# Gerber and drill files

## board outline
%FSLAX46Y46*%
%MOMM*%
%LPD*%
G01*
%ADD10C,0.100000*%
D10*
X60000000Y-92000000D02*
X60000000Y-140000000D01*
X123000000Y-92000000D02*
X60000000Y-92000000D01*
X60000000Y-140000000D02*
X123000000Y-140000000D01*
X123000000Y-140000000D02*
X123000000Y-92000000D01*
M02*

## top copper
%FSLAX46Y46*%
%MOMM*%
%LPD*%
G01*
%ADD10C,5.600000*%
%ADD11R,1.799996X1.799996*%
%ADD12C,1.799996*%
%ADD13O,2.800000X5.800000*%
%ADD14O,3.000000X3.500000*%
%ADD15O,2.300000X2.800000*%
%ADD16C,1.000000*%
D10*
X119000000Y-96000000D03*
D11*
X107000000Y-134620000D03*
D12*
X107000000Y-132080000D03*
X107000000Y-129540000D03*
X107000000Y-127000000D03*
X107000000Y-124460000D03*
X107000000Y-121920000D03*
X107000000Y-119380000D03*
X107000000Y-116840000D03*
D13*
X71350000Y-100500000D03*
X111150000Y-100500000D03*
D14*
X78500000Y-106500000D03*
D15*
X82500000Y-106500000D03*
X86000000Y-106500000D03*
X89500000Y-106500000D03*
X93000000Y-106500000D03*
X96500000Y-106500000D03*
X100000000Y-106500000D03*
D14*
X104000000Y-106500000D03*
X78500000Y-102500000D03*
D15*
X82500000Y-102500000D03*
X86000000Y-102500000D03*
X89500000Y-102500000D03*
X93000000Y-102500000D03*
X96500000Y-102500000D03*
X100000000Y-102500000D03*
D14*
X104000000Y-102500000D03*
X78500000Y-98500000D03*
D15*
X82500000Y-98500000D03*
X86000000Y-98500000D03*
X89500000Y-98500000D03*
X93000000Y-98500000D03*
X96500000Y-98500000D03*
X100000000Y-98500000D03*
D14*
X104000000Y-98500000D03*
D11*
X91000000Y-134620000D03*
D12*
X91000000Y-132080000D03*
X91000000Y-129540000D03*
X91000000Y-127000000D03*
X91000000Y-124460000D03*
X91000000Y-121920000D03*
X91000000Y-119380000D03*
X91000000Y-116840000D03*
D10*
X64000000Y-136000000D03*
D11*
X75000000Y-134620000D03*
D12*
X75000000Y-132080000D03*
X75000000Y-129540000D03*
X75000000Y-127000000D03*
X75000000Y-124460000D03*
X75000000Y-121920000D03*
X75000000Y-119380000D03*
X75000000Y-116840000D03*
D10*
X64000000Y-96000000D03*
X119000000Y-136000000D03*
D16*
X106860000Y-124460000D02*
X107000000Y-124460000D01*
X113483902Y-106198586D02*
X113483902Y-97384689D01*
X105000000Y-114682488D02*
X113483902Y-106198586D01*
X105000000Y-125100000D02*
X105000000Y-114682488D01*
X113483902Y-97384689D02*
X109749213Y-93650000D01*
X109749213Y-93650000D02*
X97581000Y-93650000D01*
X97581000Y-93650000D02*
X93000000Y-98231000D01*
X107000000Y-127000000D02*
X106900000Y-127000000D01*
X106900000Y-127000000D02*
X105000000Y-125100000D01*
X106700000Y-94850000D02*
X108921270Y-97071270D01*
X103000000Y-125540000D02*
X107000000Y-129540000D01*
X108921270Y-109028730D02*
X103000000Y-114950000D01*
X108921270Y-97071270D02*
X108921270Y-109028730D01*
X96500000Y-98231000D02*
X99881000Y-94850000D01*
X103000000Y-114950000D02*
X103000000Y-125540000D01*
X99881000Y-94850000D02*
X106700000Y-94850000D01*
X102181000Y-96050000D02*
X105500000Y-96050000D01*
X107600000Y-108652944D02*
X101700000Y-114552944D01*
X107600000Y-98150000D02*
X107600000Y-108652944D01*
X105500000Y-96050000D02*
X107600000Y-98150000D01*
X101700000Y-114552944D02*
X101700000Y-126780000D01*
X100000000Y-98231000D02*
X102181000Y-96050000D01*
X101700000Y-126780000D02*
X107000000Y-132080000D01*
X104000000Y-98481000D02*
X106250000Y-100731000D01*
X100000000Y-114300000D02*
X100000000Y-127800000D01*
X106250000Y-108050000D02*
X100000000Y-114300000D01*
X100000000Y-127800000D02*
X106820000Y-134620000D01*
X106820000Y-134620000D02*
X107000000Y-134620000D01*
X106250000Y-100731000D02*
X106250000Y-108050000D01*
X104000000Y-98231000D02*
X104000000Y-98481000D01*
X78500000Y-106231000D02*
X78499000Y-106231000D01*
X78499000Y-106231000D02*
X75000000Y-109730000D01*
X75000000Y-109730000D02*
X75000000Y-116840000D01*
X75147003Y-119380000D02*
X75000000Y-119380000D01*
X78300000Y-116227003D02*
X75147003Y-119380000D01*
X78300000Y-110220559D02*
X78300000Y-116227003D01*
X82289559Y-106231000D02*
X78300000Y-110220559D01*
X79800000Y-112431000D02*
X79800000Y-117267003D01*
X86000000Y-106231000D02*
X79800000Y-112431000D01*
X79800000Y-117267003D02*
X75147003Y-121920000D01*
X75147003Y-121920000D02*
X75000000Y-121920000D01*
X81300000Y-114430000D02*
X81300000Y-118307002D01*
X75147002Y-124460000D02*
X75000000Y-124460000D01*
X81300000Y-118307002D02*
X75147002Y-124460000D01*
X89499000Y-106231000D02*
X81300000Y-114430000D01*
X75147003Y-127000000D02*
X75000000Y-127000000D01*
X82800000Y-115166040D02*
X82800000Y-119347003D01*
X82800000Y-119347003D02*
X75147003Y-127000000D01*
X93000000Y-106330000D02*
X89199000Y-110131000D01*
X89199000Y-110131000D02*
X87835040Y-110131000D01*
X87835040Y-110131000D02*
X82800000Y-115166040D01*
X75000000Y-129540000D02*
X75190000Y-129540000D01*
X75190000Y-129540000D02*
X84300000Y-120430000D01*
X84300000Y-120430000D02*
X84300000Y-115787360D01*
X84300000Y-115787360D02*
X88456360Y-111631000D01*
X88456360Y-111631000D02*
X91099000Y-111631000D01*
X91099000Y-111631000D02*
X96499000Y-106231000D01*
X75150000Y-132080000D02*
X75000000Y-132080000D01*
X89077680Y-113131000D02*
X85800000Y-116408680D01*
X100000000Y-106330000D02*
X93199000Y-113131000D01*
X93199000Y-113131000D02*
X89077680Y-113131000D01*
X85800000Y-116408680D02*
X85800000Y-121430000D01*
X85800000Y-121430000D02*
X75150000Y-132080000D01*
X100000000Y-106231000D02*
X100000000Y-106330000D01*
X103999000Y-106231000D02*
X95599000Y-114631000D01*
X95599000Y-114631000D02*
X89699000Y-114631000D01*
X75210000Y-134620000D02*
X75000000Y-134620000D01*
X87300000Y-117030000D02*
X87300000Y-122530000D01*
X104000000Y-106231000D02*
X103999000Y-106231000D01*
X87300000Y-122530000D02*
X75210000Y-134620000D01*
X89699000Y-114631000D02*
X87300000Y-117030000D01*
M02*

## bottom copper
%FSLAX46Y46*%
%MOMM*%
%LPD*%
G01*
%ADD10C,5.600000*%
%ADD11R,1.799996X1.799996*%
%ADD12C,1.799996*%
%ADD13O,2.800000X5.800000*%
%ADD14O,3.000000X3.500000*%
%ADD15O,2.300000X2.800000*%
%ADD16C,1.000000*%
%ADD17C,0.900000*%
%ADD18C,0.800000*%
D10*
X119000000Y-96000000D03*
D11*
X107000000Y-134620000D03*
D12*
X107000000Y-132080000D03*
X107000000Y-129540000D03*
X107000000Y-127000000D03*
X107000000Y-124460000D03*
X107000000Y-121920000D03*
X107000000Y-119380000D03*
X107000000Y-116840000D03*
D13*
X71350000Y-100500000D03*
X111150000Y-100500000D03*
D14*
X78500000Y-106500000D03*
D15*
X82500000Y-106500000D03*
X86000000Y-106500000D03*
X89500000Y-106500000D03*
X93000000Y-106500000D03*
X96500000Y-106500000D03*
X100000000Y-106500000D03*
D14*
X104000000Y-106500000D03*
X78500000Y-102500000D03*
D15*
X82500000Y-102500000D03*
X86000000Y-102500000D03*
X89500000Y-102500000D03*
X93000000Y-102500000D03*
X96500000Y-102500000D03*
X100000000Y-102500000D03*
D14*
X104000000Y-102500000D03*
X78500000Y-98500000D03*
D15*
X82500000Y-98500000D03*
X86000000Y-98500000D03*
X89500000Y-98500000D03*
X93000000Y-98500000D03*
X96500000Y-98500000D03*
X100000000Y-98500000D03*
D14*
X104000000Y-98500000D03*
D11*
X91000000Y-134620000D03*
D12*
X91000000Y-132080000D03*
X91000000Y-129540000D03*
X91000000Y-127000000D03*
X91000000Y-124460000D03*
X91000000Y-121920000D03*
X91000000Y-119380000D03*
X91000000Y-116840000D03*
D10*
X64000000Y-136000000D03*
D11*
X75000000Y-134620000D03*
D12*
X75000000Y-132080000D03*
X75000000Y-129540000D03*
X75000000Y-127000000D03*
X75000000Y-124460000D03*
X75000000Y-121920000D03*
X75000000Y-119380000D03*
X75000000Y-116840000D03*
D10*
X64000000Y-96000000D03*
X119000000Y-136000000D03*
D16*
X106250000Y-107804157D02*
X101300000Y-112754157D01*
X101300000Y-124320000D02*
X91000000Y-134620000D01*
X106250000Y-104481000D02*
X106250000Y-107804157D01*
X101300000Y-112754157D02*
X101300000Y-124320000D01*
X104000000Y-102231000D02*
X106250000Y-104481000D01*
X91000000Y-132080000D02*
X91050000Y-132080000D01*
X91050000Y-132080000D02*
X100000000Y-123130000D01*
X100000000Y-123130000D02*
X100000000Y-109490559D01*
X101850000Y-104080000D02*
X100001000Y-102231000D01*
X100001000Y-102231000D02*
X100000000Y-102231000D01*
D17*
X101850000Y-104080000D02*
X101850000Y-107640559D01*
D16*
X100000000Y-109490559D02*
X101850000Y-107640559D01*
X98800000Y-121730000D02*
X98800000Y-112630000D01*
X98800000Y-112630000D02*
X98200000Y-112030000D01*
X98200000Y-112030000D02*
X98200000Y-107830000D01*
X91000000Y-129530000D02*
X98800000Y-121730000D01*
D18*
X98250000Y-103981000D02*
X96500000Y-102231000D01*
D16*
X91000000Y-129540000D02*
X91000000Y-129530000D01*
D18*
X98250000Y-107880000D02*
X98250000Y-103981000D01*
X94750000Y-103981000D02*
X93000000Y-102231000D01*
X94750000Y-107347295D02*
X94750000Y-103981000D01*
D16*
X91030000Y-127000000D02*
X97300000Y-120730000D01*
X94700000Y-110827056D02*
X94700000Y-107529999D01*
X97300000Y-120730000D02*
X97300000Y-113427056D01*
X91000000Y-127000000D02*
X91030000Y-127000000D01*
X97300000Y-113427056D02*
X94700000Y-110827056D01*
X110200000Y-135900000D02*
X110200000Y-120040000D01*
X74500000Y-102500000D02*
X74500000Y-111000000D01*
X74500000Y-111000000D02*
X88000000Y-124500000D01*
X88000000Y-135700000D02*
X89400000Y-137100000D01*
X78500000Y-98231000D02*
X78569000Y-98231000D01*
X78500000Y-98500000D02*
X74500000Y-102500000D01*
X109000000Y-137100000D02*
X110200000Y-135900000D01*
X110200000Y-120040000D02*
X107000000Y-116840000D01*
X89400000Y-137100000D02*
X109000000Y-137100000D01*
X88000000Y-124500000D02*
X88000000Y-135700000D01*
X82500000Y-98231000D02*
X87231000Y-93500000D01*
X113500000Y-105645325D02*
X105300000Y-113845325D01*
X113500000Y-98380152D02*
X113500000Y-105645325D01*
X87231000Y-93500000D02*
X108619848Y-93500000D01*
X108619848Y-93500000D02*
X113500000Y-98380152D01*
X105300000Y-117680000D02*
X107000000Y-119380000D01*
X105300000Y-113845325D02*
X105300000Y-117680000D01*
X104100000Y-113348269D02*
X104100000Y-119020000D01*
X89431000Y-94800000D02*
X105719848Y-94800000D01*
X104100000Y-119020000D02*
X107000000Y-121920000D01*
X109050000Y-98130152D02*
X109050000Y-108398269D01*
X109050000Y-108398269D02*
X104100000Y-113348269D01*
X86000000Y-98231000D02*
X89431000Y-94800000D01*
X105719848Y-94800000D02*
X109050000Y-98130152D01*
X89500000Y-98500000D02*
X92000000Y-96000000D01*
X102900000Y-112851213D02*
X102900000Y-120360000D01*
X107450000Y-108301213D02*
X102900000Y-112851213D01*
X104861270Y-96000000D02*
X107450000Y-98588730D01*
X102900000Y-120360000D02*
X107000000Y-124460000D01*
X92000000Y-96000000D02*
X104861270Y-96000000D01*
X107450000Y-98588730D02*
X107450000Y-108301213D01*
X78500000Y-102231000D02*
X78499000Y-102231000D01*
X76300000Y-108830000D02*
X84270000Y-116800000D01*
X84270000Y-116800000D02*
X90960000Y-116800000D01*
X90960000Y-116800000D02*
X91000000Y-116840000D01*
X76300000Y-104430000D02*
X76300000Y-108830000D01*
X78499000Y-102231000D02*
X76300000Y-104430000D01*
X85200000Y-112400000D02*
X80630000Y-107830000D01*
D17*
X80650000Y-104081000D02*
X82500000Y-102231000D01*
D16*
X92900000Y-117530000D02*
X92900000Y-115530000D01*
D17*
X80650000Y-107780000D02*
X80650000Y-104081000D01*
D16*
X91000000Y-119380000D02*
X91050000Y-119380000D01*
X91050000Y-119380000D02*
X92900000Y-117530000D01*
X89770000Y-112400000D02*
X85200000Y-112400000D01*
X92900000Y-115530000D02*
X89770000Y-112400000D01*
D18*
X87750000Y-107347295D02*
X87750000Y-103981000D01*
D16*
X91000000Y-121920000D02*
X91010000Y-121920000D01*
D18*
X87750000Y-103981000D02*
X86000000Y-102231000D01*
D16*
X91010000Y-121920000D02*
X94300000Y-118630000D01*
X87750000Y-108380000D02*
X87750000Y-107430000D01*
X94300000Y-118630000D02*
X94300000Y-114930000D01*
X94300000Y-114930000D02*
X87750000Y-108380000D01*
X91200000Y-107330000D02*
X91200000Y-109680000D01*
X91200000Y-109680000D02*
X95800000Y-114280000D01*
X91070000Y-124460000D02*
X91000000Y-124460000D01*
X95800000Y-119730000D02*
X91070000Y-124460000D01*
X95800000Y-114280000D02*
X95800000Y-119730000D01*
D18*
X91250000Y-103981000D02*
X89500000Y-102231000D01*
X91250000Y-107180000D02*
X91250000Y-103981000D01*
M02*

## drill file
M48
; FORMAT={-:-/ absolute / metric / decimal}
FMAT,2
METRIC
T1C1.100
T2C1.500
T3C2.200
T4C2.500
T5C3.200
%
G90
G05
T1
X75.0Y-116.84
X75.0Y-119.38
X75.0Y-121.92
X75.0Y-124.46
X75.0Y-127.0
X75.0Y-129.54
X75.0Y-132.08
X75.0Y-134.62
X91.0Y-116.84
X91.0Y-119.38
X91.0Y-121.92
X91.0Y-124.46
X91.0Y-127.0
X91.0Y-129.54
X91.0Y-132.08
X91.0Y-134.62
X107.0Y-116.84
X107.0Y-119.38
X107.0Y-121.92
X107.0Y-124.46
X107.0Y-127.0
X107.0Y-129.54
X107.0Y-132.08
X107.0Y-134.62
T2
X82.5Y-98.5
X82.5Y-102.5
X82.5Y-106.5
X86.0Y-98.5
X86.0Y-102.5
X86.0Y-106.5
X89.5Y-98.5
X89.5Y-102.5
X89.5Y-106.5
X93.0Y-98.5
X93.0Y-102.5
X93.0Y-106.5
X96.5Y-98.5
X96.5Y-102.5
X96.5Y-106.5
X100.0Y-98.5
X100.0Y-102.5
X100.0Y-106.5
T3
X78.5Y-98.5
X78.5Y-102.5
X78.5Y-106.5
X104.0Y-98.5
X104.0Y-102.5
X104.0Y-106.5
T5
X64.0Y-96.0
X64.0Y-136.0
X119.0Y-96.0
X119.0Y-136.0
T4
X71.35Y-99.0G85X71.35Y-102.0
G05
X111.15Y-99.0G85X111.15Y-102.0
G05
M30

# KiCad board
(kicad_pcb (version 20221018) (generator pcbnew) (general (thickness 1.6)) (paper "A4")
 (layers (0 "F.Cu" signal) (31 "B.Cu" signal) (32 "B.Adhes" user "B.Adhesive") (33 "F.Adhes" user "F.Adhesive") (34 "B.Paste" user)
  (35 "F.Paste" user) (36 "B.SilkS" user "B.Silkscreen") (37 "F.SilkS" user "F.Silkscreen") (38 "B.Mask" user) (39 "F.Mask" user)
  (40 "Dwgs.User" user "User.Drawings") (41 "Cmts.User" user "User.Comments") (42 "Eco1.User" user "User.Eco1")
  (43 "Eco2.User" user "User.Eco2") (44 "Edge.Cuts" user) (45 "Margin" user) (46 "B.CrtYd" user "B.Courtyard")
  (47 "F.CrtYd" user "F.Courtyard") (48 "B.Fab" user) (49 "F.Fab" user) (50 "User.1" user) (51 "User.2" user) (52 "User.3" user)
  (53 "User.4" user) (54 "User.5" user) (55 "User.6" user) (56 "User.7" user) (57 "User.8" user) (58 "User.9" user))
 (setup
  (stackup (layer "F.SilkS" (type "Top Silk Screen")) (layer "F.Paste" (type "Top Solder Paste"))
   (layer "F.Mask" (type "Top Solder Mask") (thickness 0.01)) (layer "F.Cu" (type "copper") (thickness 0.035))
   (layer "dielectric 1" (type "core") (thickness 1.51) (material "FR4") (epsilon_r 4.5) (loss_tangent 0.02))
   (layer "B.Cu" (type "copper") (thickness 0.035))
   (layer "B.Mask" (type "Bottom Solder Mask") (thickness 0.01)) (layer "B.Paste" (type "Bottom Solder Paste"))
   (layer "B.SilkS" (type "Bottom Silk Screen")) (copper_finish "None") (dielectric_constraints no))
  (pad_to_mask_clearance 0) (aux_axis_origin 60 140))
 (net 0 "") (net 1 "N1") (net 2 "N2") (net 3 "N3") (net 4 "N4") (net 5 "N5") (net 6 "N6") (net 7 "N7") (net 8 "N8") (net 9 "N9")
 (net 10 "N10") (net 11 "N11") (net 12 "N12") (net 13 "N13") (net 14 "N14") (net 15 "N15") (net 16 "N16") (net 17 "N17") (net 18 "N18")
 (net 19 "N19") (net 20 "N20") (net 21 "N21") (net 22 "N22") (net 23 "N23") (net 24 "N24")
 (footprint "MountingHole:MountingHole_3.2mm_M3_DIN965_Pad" (layer "F.Cu") (at 119 96 180)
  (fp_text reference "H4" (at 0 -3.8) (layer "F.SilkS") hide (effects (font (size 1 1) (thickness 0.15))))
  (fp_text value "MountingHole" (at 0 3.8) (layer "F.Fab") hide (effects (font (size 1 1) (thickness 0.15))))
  (pad "1" thru_hole circle (at 0 0 180) (size 5.6 5.6) (drill 3.2) (layers "*.Cu" "*.Mask")))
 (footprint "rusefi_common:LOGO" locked (layer "F.Cu") (at 67.36 115.1)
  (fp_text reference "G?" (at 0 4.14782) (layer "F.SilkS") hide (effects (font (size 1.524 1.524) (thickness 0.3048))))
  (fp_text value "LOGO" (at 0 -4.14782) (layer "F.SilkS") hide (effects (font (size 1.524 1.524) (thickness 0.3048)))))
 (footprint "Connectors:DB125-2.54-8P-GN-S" (layer "F.Cu") (at 107 125.73 90)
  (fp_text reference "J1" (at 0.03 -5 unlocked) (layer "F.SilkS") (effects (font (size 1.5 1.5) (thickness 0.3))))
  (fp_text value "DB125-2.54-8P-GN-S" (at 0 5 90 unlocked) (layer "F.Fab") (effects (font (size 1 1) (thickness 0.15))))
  (pad "1" thru_hole rect (at -8.89 0 90) (size 1.799996 1.799996) (drill 1.100023) (layers "*.Cu" "*.Mask") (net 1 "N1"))
  (pad "2" thru_hole circle (at -6.35 0 90) (size 1.799996 1.799996) (drill 1.100023) (layers "*.Cu" "*.Mask") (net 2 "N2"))
  (pad "3" thru_hole circle (at -3.81 0 90) (size 1.799996 1.799996) (drill 1.100023) (layers "*.Cu" "*.Mask") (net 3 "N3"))
  (pad "4" thru_hole circle (at -1.27 0 90) (size 1.799996 1.799996) (drill 1.100023) (layers "*.Cu" "*.Mask") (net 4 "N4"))
  (pad "5" thru_hole circle (at 1.27 0 90) (size 1.799996 1.799996) (drill 1.100023) (layers "*.Cu" "*.Mask") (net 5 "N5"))
  (pad "6" thru_hole circle (at 3.81 0 90) (size 1.799996 1.799996) (drill 1.100023) (layers "*.Cu" "*.Mask") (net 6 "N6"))
  (pad "7" thru_hole circle (at 6.35 0 90) (size 1.799996 1.799996) (drill 1.100023) (layers "*.Cu" "*.Mask") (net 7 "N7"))
  (pad "8" thru_hole circle (at 8.89 0 90) (size 1.799996 1.799996) (drill 1.100023) (layers "*.Cu" "*.Mask") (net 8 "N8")))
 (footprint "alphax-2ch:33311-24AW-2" (layer "F.Cu") (at 78.5 106.5)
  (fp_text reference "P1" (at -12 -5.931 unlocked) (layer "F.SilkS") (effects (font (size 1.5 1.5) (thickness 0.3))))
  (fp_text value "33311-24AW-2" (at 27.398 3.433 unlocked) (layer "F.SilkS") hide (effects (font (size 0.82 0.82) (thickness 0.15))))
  (pad "" thru_hole oval (at -7.15 -6 270) (size 5.8 2.8) (drill oval 5.5 2.5) (layers "*.Cu" "*.Mask") (solder_mask_margin 0.05))
  (pad "" thru_hole oval (at 32.65 -6 270) (size 5.8 2.8) (drill oval 5.5 2.5) (layers "*.Cu" "*.Mask") (solder_mask_margin 0.05))
  (pad "1" thru_hole oval (at 0 0 270) (size 3.5 3) (drill 2.2) (layers "*.Cu" "*.Mask") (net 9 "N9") (solder_mask_margin 0.05))
  (pad "2" thru_hole oval (at 4 0 270) (size 2.8 2.3) (drill 1.5) (layers "*.Cu" "*.Mask") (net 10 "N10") (solder_mask_margin 0.05))
  (pad "3" thru_hole oval (at 7.5 0 270) (size 2.8 2.3) (drill 1.5) (layers "*.Cu" "*.Mask") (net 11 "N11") (solder_mask_margin 0.05))
  (pad "4" thru_hole oval (at 11 0 270) (size 2.8 2.3) (drill 1.5) (layers "*.Cu" "*.Mask") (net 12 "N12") (solder_mask_margin 0.05))
  (pad "5" thru_hole oval (at 14.5 0 270) (size 2.8 2.3) (drill 1.5) (layers "*.Cu" "*.Mask") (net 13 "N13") (solder_mask_margin 0.05))
  (pad "6" thru_hole oval (at 18 0 270) (size 2.8 2.3) (drill 1.5) (layers "*.Cu" "*.Mask") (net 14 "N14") (solder_mask_margin 0.05))
  (pad "7" thru_hole oval (at 21.5 0 270) (size 2.8 2.3) (drill 1.5) (layers "*.Cu" "*.Mask") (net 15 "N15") (solder_mask_margin 0.05))
  (pad "8" thru_hole oval (at 25.5 0 270) (size 3.5 3) (drill 2.2) (layers "*.Cu" "*.Mask") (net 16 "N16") (solder_mask_margin 0.05))
  (pad "9" thru_hole oval (at 0 -4 270) (size 3.5 3) (drill 2.2) (layers "*.Cu" "*.Mask") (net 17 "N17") (solder_mask_margin 0.05))
  (pad "10" thru_hole oval (at 4 -4 270) (size 2.8 2.3) (drill 1.5) (layers "*.Cu" "*.Mask") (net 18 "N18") (solder_mask_margin 0.05))
  (pad "11" thru_hole oval (at 7.5 -4 270) (size 2.8 2.3) (drill 1.5) (layers "*.Cu" "*.Mask") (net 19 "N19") (solder_mask_margin 0.05))
  (pad "12" thru_hole oval (at 11 -4 270) (size 2.8 2.3) (drill 1.5) (layers "*.Cu" "*.Mask") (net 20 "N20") (solder_mask_margin 0.05))
  (pad "13" thru_hole oval (at 14.5 -4 270) (size 2.8 2.3) (drill 1.5) (layers "*.Cu" "*.Mask") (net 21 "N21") (solder_mask_margin 0.05))
  (pad "14" thru_hole oval (at 18 -4 270) (size 2.8 2.3) (drill 1.5) (layers "*.Cu" "*.Mask") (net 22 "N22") (solder_mask_margin 0.05))
  (pad "15" thru_hole oval (at 21.5 -4 270) (size 2.8 2.3) (drill 1.5) (layers "*.Cu" "*.Mask") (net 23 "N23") (solder_mask_margin 0.05))
  (pad "16" thru_hole oval (at 25.5 -4 270) (size 3.5 3) (drill 2.2) (layers "*.Cu" "*.Mask") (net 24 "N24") (solder_mask_margin 0.05))
  (pad "17" thru_hole oval (at 0 -8 270) (size 3.5 3) (drill 2.2) (layers "*.Cu" "*.Mask") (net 8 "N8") (solder_mask_margin 0.05))
  (pad "18" thru_hole oval (at 4 -8 270) (size 2.8 2.3) (drill 1.5) (layers "*.Cu" "*.Mask") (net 7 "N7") (solder_mask_margin 0.05))
  (pad "19" thru_hole oval (at 7.5 -8 270) (size 2.8 2.3) (drill 1.5) (layers "*.Cu" "*.Mask") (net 6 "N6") (solder_mask_margin 0.05))
  (pad "20" thru_hole oval (at 11 -8 270) (size 2.8 2.3) (drill 1.5) (layers "*.Cu" "*.Mask") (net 5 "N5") (solder_mask_margin 0.05))
  (pad "21" thru_hole oval (at 14.5 -8 270) (size 2.8 2.3) (drill 1.5) (layers "*.Cu" "*.Mask") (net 4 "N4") (solder_mask_margin 0.05))
  (pad "22" thru_hole oval (at 18 -8 270) (size 2.8 2.3) (drill 1.5) (layers "*.Cu" "*.Mask") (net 3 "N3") (solder_mask_margin 0.05))
  (pad "23" thru_hole oval (at 21.5 -8 270) (size 2.8 2.3) (drill 1.5) (layers "*.Cu" "*.Mask") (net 2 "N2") (solder_mask_margin 0.05))
  (pad "24" thru_hole oval (at 25.5 -8 270) (size 3.5 3) (drill 2.2) (layers "*.Cu" "*.Mask") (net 1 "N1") (solder_mask_margin 0.05)))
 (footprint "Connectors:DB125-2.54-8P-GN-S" (layer "F.Cu") (at 91 125.73 90)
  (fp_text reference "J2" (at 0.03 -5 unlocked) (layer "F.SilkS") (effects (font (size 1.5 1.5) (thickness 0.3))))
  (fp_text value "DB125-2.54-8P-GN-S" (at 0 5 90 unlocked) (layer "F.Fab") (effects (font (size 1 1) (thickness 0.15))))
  (pad "1" thru_hole rect (at -8.89 0 90) (size 1.799996 1.799996) (drill 1.100023) (layers "*.Cu" "*.Mask") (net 24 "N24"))
  (pad "2" thru_hole circle (at -6.35 0 90) (size 1.799996 1.799996) (drill 1.100023) (layers "*.Cu" "*.Mask") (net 23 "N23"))
  (pad "3" thru_hole circle (at -3.81 0 90) (size 1.799996 1.799996) (drill 1.100023) (layers "*.Cu" "*.Mask") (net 22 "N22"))
  (pad "4" thru_hole circle (at -1.27 0 90) (size 1.799996 1.799996) (drill 1.100023) (layers "*.Cu" "*.Mask") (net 21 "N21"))
  (pad "5" thru_hole circle (at 1.27 0 90) (size 1.799996 1.799996) (drill 1.100023) (layers "*.Cu" "*.Mask") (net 20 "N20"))
  (pad "6" thru_hole circle (at 3.81 0 90) (size 1.799996 1.799996) (drill 1.100023) (layers "*.Cu" "*.Mask") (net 19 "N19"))
  (pad "7" thru_hole circle (at 6.35 0 90) (size 1.799996 1.799996) (drill 1.100023) (layers "*.Cu" "*.Mask") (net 18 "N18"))
  (pad "8" thru_hole circle (at 8.89 0 90) (size 1.799996 1.799996) (drill 1.100023) (layers "*.Cu" "*.Mask") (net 17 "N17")))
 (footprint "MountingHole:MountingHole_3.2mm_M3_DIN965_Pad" (layer "F.Cu") (at 64 136 180)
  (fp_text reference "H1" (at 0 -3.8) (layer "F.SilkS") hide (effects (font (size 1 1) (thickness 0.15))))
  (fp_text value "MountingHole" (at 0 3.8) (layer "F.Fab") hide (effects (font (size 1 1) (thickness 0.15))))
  (pad "1" thru_hole circle (at 0 0 180) (size 5.6 5.6) (drill 3.2) (layers "*.Cu" "*.Mask")))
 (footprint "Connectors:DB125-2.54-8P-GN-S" (layer "F.Cu") (at 75 125.73 90)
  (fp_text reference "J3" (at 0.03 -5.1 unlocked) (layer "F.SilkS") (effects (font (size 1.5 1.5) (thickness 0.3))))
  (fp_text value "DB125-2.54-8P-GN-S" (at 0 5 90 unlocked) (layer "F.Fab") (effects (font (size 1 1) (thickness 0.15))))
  (pad "1" thru_hole rect (at -8.89 0 90) (size 1.799996 1.799996) (drill 1.100023) (layers "*.Cu" "*.Mask") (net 16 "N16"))
  (pad "2" thru_hole circle (at -6.35 0 90) (size 1.799996 1.799996) (drill 1.100023) (layers "*.Cu" "*.Mask") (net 15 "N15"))
  (pad "3" thru_hole circle (at -3.81 0 90) (size 1.799996 1.799996) (drill 1.100023) (layers "*.Cu" "*.Mask") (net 14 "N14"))
  (pad "4" thru_hole circle (at -1.27 0 90) (size 1.799996 1.799996) (drill 1.100023) (layers "*.Cu" "*.Mask") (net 13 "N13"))
  (pad "5" thru_hole circle (at 1.27 0 90) (size 1.799996 1.799996) (drill 1.100023) (layers "*.Cu" "*.Mask") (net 12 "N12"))
  (pad "6" thru_hole circle (at 3.81 0 90) (size 1.799996 1.799996) (drill 1.100023) (layers "*.Cu" "*.Mask") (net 11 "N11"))
  (pad "7" thru_hole circle (at 6.35 0 90) (size 1.799996 1.799996) (drill 1.100023) (layers "*.Cu" "*.Mask") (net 10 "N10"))
  (pad "8" thru_hole circle (at 8.89 0 90) (size 1.799996 1.799996) (drill 1.100023) (layers "*.Cu" "*.Mask") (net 9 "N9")))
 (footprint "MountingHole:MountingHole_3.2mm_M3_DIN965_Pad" (layer "F.Cu") (at 64 96 180)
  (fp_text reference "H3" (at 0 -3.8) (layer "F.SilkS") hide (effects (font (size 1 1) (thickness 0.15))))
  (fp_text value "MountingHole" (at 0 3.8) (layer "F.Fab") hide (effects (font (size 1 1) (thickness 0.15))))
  (pad "1" thru_hole circle (at 0 0 180) (size 5.6 5.6) (drill 3.2) (layers "*.Cu" "*.Mask")))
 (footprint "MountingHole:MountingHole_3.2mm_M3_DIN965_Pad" (layer "F.Cu") (at 119 136 180)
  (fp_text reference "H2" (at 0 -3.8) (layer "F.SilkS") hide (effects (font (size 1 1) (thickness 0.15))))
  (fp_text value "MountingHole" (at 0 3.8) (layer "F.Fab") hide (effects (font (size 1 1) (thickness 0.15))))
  (pad "1" thru_hole circle (at 0 0 180) (size 5.6 5.6) (drill 3.2) (layers "*.Cu" "*.Mask")))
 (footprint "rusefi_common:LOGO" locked (layer "B.Cu") (at 114.934286 115.2 180)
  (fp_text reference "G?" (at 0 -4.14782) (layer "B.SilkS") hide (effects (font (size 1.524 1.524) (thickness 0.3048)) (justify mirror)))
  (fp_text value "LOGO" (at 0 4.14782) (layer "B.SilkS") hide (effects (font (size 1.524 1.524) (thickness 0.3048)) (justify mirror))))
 (gr_line (start 60 92) (end 60 140) (stroke (width 0.1) (type solid)) (layer "Edge.Cuts"))
 (gr_line (start 123 92) (end 60 92) (stroke (width 0.1) (type solid)) (layer "Edge.Cuts"))
 (gr_line (start 60 140) (end 123 140) (stroke (width 0.1) (type solid)) (layer "Edge.Cuts"))
 (gr_line (start 123 140) (end 123 92) (stroke (width 0.1) (type solid)) (layer "Edge.Cuts"))
 (segment (start 106.25 107.804157) (end 101.3 112.754157) (width 1) (layer "B.Cu") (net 24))
 (segment (start 101.3 124.32) (end 91 134.62) (width 1) (layer "B.Cu") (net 24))
 (segment (start 106.25 104.481) (end 106.25 107.804157) (width 1) (layer "B.Cu") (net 24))
 (segment (start 101.3 112.754157) (end 101.3 124.32) (width 1) (layer "B.Cu") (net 24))
 (segment (start 104 102.231) (end 106.25 104.481) (width 1) (layer "B.Cu") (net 24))
 (segment (start 91 132.08) (end 91.05 132.08) (width 1) (layer "B.Cu") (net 23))
 (segment (start 91.05 132.08) (end 100 123.13) (width 1) (layer "B.Cu") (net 23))
 (segment (start 100 123.13) (end 100 109.490559) (width 1) (layer "B.Cu") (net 23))
 (segment (start 101.85 104.08) (end 100.001 102.231) (width 1) (layer "B.Cu") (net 23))
 (segment (start 100.001 102.231) (end 100 102.231) (width 1) (layer "B.Cu") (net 23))
 (segment (start 101.85 104.08) (end 101.85 107.640559) (width 0.9) (layer "B.Cu") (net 23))
 (segment (start 100 109.490559) (end 101.85 107.640559) (width 1) (layer "B.Cu") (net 23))
 (segment (start 98.8 121.73) (end 98.8 112.63) (width 1) (layer "B.Cu") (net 22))
 (segment (start 98.8 112.63) (end 98.2 112.03) (width 1) (layer "B.Cu") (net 22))
 (segment (start 98.2 112.03) (end 98.2 107.83) (width 1) (layer "B.Cu") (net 22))
 (segment (start 91 129.53) (end 98.8 121.73) (width 1) (layer "B.Cu") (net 22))
 (segment (start 98.25 103.981) (end 96.5 102.231) (width 0.8) (layer "B.Cu") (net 22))
 (segment (start 91 129.54) (end 91 129.53) (width 1) (layer "B.Cu") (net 22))
 (segment (start 98.25 107.88) (end 98.25 103.981) (width 0.8) (layer "B.Cu") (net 22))
 (segment (start 94.75 103.981) (end 93 102.231) (width 0.8) (layer "B.Cu") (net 21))
 (segment (start 94.75 107.347295) (end 94.75 103.981) (width 0.8) (layer "B.Cu") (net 21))
 (segment (start 91.03 127) (end 97.3 120.73) (width 1) (layer "B.Cu") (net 21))
 (segment (start 94.7 110.827056) (end 94.7 107.529999) (width 1) (layer "B.Cu") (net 21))
 (segment (start 97.3 120.73) (end 97.3 113.427056) (width 1) (layer "B.Cu") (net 21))
 (segment (start 91 127) (end 91.03 127) (width 1) (layer "B.Cu") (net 21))
 (segment (start 97.3 113.427056) (end 94.7 110.827056) (width 1) (layer "B.Cu") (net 21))
 (segment (start 110.2 135.9) (end 110.2 120.04) (width 1) (layer "B.Cu") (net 8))
 (segment (start 74.5 102.5) (end 74.5 111) (width 1) (layer "B.Cu") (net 8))
 (segment (start 74.5 111) (end 88 124.5) (width 1) (layer "B.Cu") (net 8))
 (segment (start 88 135.7) (end 89.4 137.1) (width 1) (layer "B.Cu") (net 8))
 (segment (start 78.5 98.231) (end 78.569 98.231) (width 1) (layer "B.Cu") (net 8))
 (segment (start 78.5 98.5) (end 74.5 102.5) (width 1) (layer "B.Cu") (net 8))
 (segment (start 109 137.1) (end 110.2 135.9) (width 1) (layer "B.Cu") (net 8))
 (segment (start 110.2 120.04) (end 107 116.84) (width 1) (layer "B.Cu") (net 8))
 (segment (start 89.4 137.1) (end 109 137.1) (width 1) (layer "B.Cu") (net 8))
 (segment (start 88 124.5) (end 88 135.7) (width 1) (layer "B.Cu") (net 8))
 (segment (start 82.5 98.231) (end 87.231 93.5) (width 1) (layer "B.Cu") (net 7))
 (segment (start 113.5 105.645325) (end 105.3 113.845325) (width 1) (layer "B.Cu") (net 7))
 (segment (start 113.5 98.380152) (end 113.5 105.645325) (width 1) (layer "B.Cu") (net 7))
 (segment (start 87.231 93.5) (end 108.619848 93.5) (width 1) (layer "B.Cu") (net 7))
 (segment (start 108.619848 93.5) (end 113.5 98.380152) (width 1) (layer "B.Cu") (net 7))
 (segment (start 105.3 117.68) (end 107 119.38) (width 1) (layer "B.Cu") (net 7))
 (segment (start 105.3 113.845325) (end 105.3 117.68) (width 1) (layer "B.Cu") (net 7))
 (segment (start 104.1 113.348269) (end 104.1 119.02) (width 1) (layer "B.Cu") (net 6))
 (segment (start 89.431 94.8) (end 105.719848 94.8) (width 1) (layer "B.Cu") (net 6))
 (segment (start 104.1 119.02) (end 107 121.92) (width 1) (layer "B.Cu") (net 6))
 (segment (start 109.05 98.130152) (end 109.05 108.398269) (width 1) (layer "B.Cu") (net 6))
 (segment (start 109.05 108.398269) (end 104.1 113.348269) (width 1) (layer "B.Cu") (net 6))
 (segment (start 86 98.231) (end 89.431 94.8) (width 1) (layer "B.Cu") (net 6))
 (segment (start 105.719848 94.8) (end 109.05 98.130152) (width 1) (layer "B.Cu") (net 6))
 (segment (start 106.86 124.46) (end 107 124.46) (width 1) (layer "F.Cu") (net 5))
 (segment (start 89.5 98.5) (end 92 96) (width 1) (layer "B.Cu") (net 5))
 (segment (start 102.9 112.851213) (end 102.9 120.36) (width 1) (layer "B.Cu") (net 5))
 (segment (start 107.45 108.301213) (end 102.9 112.851213) (width 1) (layer "B.Cu") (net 5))
 (segment (start 104.86127 96) (end 107.45 98.58873) (width 1) (layer "B.Cu") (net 5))
 (segment (start 102.9 120.36) (end 107 124.46) (width 1) (layer "B.Cu") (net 5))
 (segment (start 92 96) (end 104.86127 96) (width 1) (layer "B.Cu") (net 5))
 (segment (start 107.45 98.58873) (end 107.45 108.301213) (width 1) (layer "B.Cu") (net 5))
 (segment (start 113.483902 106.198586) (end 113.483902 97.384689) (width 1) (layer "F.Cu") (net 4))
 (segment (start 105 114.682488) (end 113.483902 106.198586) (width 1) (layer "F.Cu") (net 4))
 (segment (start 105 125.1) (end 105 114.682488) (width 1) (layer "F.Cu") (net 4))
 (segment (start 113.483902 97.384689) (end 109.749213 93.65) (width 1) (layer "F.Cu") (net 4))
 (segment (start 109.749213 93.65) (end 97.581 93.65) (width 1) (layer "F.Cu") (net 4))
 (segment (start 97.581 93.65) (end 93 98.231) (width 1) (layer "F.Cu") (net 4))
 (segment (start 107 127) (end 106.9 127) (width 1) (layer "F.Cu") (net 4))
 (segment (start 106.9 127) (end 105 125.1) (width 1) (layer "F.Cu") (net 4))
 (segment (start 106.7 94.85) (end 108.92127 97.07127) (width 1) (layer "F.Cu") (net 3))
 (segment (start 103 125.54) (end 107 129.54) (width 1) (layer "F.Cu") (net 3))
 (segment (start 108.92127 109.02873) (end 103 114.95) (width 1) (layer "F.Cu") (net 3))
 (segment (start 108.92127 97.07127) (end 108.92127 109.02873) (width 1) (layer "F.Cu") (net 3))
 (segment (start 96.5 98.231) (end 99.881 94.85) (width 1) (layer "F.Cu") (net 3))
 (segment (start 103 114.95) (end 103 125.54) (width 1) (layer "F.Cu") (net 3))
 (segment (start 99.881 94.85) (end 106.7 94.85) (width 1) (layer "F.Cu") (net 3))
 (segment (start 102.181 96.05) (end 105.5 96.05) (width 1) (layer "F.Cu") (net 2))
 (segment (start 107.6 108.652944) (end 101.7 114.552944) (width 1) (layer "F.Cu") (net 2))
 (segment (start 107.6 98.15) (end 107.6 108.652944) (width 1) (layer "F.Cu") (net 2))
 (segment (start 105.5 96.05) (end 107.6 98.15) (width 1) (layer "F.Cu") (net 2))
 (segment (start 101.7 114.552944) (end 101.7 126.78) (width 1) (layer "F.Cu") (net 2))
 (segment (start 100 98.231) (end 102.181 96.05) (width 1) (layer "F.Cu") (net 2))
 (segment (start 101.7 126.78) (end 107 132.08) (width 1) (layer "F.Cu") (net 2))
 (segment (start 104 98.481) (end 106.25 100.731) (width 1) (layer "F.Cu") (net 1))
 (segment (start 100 114.3) (end 100 127.8) (width 1) (layer "F.Cu") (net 1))
 (segment (start 106.25 108.05) (end 100 114.3) (width 1) (layer "F.Cu") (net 1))
 (segment (start 100 127.8) (end 106.82 134.62) (width 1) (layer "F.Cu") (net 1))
 (segment (start 106.82 134.62) (end 107 134.62) (width 1) (layer "F.Cu") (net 1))
 (segment (start 106.25 100.731) (end 106.25 108.05) (width 1) (layer "F.Cu") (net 1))
 (segment (start 104 98.231) (end 104 98.481) (width 1) (layer "F.Cu") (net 1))
 (segment (start 78.5 102.231) (end 78.499 102.231) (width 1) (layer "B.Cu") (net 17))
 (segment (start 76.3 108.83) (end 84.27 116.8) (width 1) (layer "B.Cu") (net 17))
 (segment (start 84.27 116.8) (end 90.96 116.8) (width 1) (layer "B.Cu") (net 17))
 (segment (start 90.96 116.8) (end 91 116.84) (width 1) (layer "B.Cu") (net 17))
 (segment (start 76.3 104.43) (end 76.3 108.83) (width 1) (layer "B.Cu") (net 17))
 (segment (start 78.499 102.231) (end 76.3 104.43) (width 1) (layer "B.Cu") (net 17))
 (segment (start 85.2 112.4) (end 80.63 107.83) (width 1) (layer "B.Cu") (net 18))
 (segment (start 80.65 104.081) (end 82.5 102.231) (width 0.9) (layer "B.Cu") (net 18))
 (segment (start 92.9 117.53) (end 92.9 115.53) (width 1) (layer "B.Cu") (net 18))
 (segment (start 80.65 107.78) (end 80.65 104.081) (width 0.9) (layer "B.Cu") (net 18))
 (segment (start 91 119.38) (end 91.05 119.38) (width 1) (layer "B.Cu") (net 18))
 (segment (start 91.05 119.38) (end 92.9 117.53) (width 1) (layer "B.Cu") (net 18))
 (segment (start 89.77 112.4) (end 85.2 112.4) (width 1) (layer "B.Cu") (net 18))
 (segment (start 92.9 115.53) (end 89.77 112.4) (width 1) (layer "B.Cu") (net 18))
 (segment (start 87.75 107.347295) (end 87.75 103.981) (width 0.8) (layer "B.Cu") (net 19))
 (segment (start 91 121.92) (end 91.01 121.92) (width 1) (layer "B.Cu") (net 19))
 (segment (start 87.75 103.981) (end 86 102.231) (width 0.8) (layer "B.Cu") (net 19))
 (segment (start 91.01 121.92) (end 94.3 118.63) (width 1) (layer "B.Cu") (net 19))
 (segment (start 87.75 108.38) (end 87.75 107.43) (width 1) (layer "B.Cu") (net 19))
 (segment (start 94.3 118.63) (end 94.3 114.93) (width 1) (layer "B.Cu") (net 19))
 (segment (start 94.3 114.93) (end 87.75 108.38) (width 1) (layer "B.Cu") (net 19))
 (segment (start 91.2 107.33) (end 91.2 109.68) (width 1) (layer "B.Cu") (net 20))
 (segment (start 91.2 109.68) (end 95.8 114.28) (width 1) (layer "B.Cu") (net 20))
 (segment (start 91.07 124.46) (end 91 124.46) (width 1) (layer "B.Cu") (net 20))
 (segment (start 95.8 119.73) (end 91.07 124.46) (width 1) (layer "B.Cu") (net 20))
 (segment (start 95.8 114.28) (end 95.8 119.73) (width 1) (layer "B.Cu") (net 20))
 (segment (start 91.25 103.981) (end 89.5 102.231) (width 0.8) (layer "B.Cu") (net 20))
 (segment (start 91.25 107.18) (end 91.25 103.981) (width 0.8) (layer "B.Cu") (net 20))
 (segment (start 78.5 106.231) (end 78.499 106.231) (width 1) (layer "F.Cu") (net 9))
 (segment (start 78.499 106.231) (end 75 109.73) (width 1) (layer "F.Cu") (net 9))
 (segment (start 75 109.73) (end 75 116.84) (width 1) (layer "F.Cu") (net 9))
 (segment (start 75.147003 119.38) (end 75 119.38) (width 1) (layer "F.Cu") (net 10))
 (segment (start 78.3 116.227003) (end 75.147003 119.38) (width 1) (layer "F.Cu") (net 10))
 (segment (start 78.3 110.220559) (end 78.3 116.227003) (width 1) (layer "F.Cu") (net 10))
 (segment (start 82.289559 106.231) (end 78.3 110.220559) (width 1) (layer "F.Cu") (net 10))
 (segment (start 79.8 112.431) (end 79.8 117.267003) (width 1) (layer "F.Cu") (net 11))
 (segment (start 86 106.231) (end 79.8 112.431) (width 1) (layer "F.Cu") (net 11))
 (segment (start 79.8 117.267003) (end 75.147003 121.92) (width 1) (layer "F.Cu") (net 11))
 (segment (start 75.147003 121.92) (end 75 121.92) (width 1) (layer "F.Cu") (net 11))
 (segment (start 81.3 114.43) (end 81.3 118.307002) (width 1) (layer "F.Cu") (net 12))
 (segment (start 75.147002 124.46) (end 75 124.46) (width 1) (layer "F.Cu") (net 12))
 (segment (start 81.3 118.307002) (end 75.147002 124.46) (width 1) (layer "F.Cu") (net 12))
 (segment (start 89.499 106.231) (end 81.3 114.43) (width 1) (layer "F.Cu") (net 12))
 (segment (start 75.147003 127) (end 75 127) (width 1) (layer "F.Cu") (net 13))
 (segment (start 82.8 115.16604) (end 82.8 119.347003) (width 1) (layer "F.Cu") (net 13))
 (segment (start 82.8 119.347003) (end 75.147003 127) (width 1) (layer "F.Cu") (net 13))
 (segment (start 93 106.33) (end 89.199 110.131) (width 1) (layer "F.Cu") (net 13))
 (segment (start 89.199 110.131) (end 87.83504 110.131) (width 1) (layer "F.Cu") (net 13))
 (segment (start 87.83504 110.131) (end 82.8 115.16604) (width 1) (layer "F.Cu") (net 13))
 (segment (start 75 129.54) (end 75.19 129.54) (width 1) (layer "F.Cu") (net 14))
 (segment (start 75.19 129.54) (end 84.3 120.43) (width 1) (layer "F.Cu") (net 14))
 (segment (start 84.3 120.43) (end 84.3 115.78736) (width 1) (layer "F.Cu") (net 14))
 (segment (start 84.3 115.78736) (end 88.45636 111.631) (width 1) (layer "F.Cu") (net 14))
 (segment (start 88.45636 111.631) (end 91.099 111.631) (width 1) (layer "F.Cu") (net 14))
 (segment (start 91.099 111.631) (end 96.499 106.231) (width 1) (layer "F.Cu") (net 14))
 (segment (start 75.15 132.08) (end 75 132.08) (width 1) (layer "F.Cu") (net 15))
 (segment (start 89.07768 113.131) (end 85.8 116.40868) (width 1) (layer "F.Cu") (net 15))
 (segment (start 100 106.33) (end 93.199 113.131) (width 1) (layer "F.Cu") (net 15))
 (segment (start 93.199 113.131) (end 89.07768 113.131) (width 1) (layer "F.Cu") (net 15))
 (segment (start 85.8 116.40868) (end 85.8 121.43) (width 1) (layer "F.Cu") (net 15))
 (segment (start 85.8 121.43) (end 75.15 132.08) (width 1) (layer "F.Cu") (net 15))
 (segment (start 100 106.231) (end 100 106.33) (width 1) (layer "F.Cu") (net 15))
 (segment (start 103.999 106.231) (end 95.599 114.631) (width 1) (layer "F.Cu") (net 16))
 (segment (start 95.599 114.631) (end 89.699 114.631) (width 1) (layer "F.Cu") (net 16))
 (segment (start 75.21 134.62) (end 75 134.62) (width 1) (layer "F.Cu") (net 16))
 (segment (start 87.3 117.03) (end 87.3 122.53) (width 1) (layer "F.Cu") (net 16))
 (segment (start 104 106.231) (end 103.999 106.231) (width 1) (layer "F.Cu") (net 16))
 (segment (start 87.3 122.53) (end 75.21 134.62) (width 1) (layer "F.Cu") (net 16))
 (segment (start 89.699 114.631) (end 87.3 117.03) (width 1) (layer "F.Cu") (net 16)))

